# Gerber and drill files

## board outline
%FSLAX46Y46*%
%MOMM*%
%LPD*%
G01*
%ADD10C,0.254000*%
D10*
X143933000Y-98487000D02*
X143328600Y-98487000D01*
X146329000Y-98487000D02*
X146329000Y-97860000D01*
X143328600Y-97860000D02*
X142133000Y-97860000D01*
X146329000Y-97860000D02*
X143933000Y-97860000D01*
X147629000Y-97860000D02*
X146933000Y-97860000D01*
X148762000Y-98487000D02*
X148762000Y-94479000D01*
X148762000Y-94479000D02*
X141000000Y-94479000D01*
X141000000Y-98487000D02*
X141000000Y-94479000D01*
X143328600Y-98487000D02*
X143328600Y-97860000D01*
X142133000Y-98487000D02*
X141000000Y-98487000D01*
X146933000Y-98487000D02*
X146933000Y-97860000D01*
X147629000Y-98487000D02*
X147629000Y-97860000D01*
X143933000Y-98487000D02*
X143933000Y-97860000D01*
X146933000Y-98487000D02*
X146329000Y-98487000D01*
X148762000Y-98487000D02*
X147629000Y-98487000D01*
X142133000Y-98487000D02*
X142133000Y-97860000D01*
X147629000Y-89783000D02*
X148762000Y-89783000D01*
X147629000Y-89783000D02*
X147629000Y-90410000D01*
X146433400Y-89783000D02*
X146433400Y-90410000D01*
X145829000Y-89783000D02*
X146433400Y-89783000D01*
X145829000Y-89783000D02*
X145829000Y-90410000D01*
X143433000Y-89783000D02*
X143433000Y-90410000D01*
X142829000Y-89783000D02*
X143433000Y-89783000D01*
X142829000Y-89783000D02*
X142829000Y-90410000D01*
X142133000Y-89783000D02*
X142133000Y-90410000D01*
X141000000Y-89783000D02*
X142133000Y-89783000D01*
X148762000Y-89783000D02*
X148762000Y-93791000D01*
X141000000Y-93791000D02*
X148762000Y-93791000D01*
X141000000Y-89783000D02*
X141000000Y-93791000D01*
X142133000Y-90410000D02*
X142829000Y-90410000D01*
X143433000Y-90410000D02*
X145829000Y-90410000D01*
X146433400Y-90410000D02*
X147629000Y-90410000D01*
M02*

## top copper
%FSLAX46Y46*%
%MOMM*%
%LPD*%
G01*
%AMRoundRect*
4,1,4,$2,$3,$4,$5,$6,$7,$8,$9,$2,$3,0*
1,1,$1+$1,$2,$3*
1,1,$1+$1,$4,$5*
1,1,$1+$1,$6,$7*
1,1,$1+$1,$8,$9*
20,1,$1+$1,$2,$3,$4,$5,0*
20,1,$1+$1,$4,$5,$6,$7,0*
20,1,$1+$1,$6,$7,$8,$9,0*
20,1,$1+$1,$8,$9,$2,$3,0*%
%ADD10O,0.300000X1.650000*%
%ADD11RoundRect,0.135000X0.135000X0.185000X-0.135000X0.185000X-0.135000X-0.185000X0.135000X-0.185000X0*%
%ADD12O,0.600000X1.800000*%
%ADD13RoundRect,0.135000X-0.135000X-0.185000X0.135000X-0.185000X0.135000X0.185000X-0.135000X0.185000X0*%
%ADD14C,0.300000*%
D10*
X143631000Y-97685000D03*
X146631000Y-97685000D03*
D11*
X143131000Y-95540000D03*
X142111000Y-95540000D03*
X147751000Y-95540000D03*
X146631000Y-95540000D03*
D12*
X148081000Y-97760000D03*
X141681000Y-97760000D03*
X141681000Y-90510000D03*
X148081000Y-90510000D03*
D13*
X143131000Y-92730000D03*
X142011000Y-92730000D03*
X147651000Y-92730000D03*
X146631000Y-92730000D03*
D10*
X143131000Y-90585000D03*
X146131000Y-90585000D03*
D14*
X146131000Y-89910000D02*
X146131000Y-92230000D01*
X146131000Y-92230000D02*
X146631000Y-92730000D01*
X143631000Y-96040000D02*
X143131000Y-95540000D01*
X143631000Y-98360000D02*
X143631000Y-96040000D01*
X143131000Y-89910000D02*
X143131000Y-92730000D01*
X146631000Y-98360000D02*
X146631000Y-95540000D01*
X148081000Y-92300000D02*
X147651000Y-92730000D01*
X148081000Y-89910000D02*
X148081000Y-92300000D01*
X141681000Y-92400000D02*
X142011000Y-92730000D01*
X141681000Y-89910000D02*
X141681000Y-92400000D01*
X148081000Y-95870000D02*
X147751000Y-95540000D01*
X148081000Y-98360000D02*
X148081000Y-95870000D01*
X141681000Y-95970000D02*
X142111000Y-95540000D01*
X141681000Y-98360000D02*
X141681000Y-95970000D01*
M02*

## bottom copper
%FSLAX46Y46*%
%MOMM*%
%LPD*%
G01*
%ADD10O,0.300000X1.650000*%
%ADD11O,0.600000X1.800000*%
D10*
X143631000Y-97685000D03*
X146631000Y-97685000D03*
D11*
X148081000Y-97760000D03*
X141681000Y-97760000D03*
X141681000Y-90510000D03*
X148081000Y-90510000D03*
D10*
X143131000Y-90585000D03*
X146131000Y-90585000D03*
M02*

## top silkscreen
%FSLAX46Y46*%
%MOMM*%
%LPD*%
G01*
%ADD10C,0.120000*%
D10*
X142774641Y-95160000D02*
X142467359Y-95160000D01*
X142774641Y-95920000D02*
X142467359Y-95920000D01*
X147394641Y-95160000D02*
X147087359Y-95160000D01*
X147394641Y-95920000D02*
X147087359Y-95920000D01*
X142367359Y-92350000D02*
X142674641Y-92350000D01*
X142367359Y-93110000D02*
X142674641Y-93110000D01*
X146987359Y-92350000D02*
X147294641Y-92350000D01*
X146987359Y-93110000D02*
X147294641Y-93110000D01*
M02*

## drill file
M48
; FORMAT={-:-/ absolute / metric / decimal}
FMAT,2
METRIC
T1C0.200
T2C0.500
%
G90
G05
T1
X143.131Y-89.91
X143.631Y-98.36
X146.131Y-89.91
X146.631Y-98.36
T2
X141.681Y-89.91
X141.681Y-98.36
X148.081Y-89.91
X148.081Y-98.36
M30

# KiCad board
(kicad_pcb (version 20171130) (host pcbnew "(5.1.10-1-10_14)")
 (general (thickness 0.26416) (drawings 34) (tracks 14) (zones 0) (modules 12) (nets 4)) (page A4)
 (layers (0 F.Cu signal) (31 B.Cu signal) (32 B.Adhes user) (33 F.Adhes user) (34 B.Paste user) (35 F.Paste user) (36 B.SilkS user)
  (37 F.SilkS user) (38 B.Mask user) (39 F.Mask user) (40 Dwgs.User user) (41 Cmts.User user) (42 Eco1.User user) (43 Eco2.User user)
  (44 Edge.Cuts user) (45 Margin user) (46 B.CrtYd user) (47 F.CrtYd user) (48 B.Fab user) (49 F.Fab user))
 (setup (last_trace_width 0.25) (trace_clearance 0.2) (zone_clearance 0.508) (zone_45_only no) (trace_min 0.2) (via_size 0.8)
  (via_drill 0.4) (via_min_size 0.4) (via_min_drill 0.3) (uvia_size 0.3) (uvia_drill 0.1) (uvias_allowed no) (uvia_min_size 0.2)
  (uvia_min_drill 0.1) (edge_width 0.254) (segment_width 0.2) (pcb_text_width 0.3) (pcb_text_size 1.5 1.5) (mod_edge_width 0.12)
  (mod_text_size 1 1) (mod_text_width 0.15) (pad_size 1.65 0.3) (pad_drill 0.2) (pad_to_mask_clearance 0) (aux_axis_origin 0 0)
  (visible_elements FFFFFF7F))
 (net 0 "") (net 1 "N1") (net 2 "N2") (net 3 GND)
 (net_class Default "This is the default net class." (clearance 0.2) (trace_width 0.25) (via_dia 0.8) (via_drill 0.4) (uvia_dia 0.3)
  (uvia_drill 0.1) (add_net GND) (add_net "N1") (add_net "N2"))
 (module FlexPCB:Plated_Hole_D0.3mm (layer F.Cu) (at 142.941 95.36 90)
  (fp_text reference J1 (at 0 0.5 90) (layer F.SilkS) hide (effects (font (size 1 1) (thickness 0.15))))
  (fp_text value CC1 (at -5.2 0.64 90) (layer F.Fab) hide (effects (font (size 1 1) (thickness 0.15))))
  (pad A5 thru_hole oval (at -3 0.69 90) (size 1.65 0.3) (drill 0.2 (offset 0.675 0)) (layers *.Cu *.Mask) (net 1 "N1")))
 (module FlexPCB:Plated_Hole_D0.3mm (layer F.Cu) (at 149.161 95.36 90)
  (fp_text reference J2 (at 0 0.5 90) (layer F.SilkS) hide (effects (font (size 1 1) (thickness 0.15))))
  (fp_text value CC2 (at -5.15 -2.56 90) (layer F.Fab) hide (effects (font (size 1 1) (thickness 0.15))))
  (pad B5 thru_hole oval (at -3 -2.53 90) (size 1.65 0.3) (drill 0.2 (offset 0.675 0)) (layers *.Cu *.Mask) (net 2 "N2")))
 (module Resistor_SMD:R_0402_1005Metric (layer F.Cu) (at 142.621 95.54 180)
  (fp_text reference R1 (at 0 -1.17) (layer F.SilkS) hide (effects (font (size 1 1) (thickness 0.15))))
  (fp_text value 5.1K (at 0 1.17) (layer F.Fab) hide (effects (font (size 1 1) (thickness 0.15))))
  (fp_line (start -0.153641 0.38) (end 0.153641 0.38) (layer F.SilkS) (width 0.12))
  (fp_line (start -0.153641 -0.38) (end 0.153641 -0.38) (layer F.SilkS) (width 0.12))
  (pad 1 smd roundrect (at -0.51 0 180) (size 0.54 0.64) (layers F.Cu F.Paste F.Mask) (roundrect_rratio 0.25) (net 1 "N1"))
  (pad 2 smd roundrect (at 0.51 0 180) (size 0.54 0.64) (layers F.Cu F.Paste F.Mask) (roundrect_rratio 0.25) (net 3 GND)))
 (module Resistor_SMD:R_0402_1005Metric (layer F.Cu) (at 147.241 95.54 180)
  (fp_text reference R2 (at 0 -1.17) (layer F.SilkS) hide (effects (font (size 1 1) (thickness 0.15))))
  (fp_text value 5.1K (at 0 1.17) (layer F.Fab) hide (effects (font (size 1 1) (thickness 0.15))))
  (fp_line (start -0.153641 0.38) (end 0.153641 0.38) (layer F.SilkS) (width 0.12))
  (fp_line (start -0.153641 -0.38) (end 0.153641 -0.38) (layer F.SilkS) (width 0.12))
  (pad 1 smd roundrect (at -0.51 0 180) (size 0.54 0.64) (layers F.Cu F.Paste F.Mask) (roundrect_rratio 0.25) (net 3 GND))
  (pad 2 smd roundrect (at 0.61 0 180) (size 0.54 0.64) (layers F.Cu F.Paste F.Mask) (roundrect_rratio 0.25) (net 2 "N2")))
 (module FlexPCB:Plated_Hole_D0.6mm (layer F.Cu) (at 146.111 99.52 180)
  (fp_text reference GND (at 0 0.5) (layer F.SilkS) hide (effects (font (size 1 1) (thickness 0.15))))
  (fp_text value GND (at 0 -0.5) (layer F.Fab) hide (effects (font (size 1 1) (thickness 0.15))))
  (pad B1 thru_hole oval (at -1.97 1.16 90) (size 1.8 0.6) (drill 0.5 (offset 0.6 0)) (layers *.Cu *.Mask) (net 3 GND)))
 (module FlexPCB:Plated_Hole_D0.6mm (layer F.Cu) (at 138.771 99.66 180)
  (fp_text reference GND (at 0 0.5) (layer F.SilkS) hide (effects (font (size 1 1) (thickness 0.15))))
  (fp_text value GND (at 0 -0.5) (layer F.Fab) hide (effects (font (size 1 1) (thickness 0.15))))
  (pad A1 thru_hole oval (at -2.91 1.3 90) (size 1.8 0.6) (drill 0.5 (offset 0.6 0)) (layers *.Cu *.Mask) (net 3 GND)))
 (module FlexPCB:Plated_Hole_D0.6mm (layer F.Cu) (at 143.651 88.75)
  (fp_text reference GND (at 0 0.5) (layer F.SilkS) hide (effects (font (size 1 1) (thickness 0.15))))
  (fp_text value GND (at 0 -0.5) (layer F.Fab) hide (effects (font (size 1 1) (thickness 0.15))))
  (pad B1 thru_hole oval (at -1.97 1.16 270) (size 1.8 0.6) (drill 0.5 (offset 0.6 0)) (layers *.Cu *.Mask) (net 3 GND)))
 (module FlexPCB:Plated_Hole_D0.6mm (layer F.Cu) (at 150.991 88.61)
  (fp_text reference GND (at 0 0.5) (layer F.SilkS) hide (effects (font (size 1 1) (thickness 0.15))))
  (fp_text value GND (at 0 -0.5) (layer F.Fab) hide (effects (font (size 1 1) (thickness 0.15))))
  (pad A1 thru_hole oval (at -2.91 1.3 270) (size 1.8 0.6) (drill 0.5 (offset 0.6 0)) (layers *.Cu *.Mask) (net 3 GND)))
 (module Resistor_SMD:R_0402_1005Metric (layer F.Cu) (at 142.521 92.73)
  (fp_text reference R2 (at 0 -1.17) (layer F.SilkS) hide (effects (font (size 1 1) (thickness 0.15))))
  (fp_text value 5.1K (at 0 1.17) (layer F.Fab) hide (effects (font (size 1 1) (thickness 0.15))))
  (fp_line (start -0.153641 -0.38) (end 0.153641 -0.38) (layer F.SilkS) (width 0.12))
  (fp_line (start -0.153641 0.38) (end 0.153641 0.38) (layer F.SilkS) (width 0.12))
  (pad 2 smd roundrect (at 0.61 0) (size 0.54 0.64) (layers F.Cu F.Paste F.Mask) (roundrect_rratio 0.25) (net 2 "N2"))
  (pad 1 smd roundrect (at -0.51 0) (size 0.54 0.64) (layers F.Cu F.Paste F.Mask) (roundrect_rratio 0.25) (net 3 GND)))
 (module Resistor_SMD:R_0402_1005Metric (layer F.Cu) (at 147.141 92.73)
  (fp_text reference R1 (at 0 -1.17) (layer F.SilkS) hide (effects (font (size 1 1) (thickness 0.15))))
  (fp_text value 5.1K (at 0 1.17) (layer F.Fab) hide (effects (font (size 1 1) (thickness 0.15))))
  (fp_line (start -0.153641 -0.38) (end 0.153641 -0.38) (layer F.SilkS) (width 0.12))
  (fp_line (start -0.153641 0.38) (end 0.153641 0.38) (layer F.SilkS) (width 0.12))
  (pad 2 smd roundrect (at 0.51 0) (size 0.54 0.64) (layers F.Cu F.Paste F.Mask) (roundrect_rratio 0.25) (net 3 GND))
  (pad 1 smd roundrect (at -0.51 0) (size 0.54 0.64) (layers F.Cu F.Paste F.Mask) (roundrect_rratio 0.25) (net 1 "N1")))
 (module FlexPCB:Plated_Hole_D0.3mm (layer F.Cu) (at 140.601 92.91 270)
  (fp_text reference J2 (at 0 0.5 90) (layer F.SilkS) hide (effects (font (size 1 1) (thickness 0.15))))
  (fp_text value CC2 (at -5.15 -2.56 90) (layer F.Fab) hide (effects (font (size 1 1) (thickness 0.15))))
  (pad B5 thru_hole oval (at -3 -2.53 270) (size 1.65 0.3) (drill 0.2 (offset 0.675 0)) (layers *.Cu *.Mask) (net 2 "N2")))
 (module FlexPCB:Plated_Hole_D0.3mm (layer F.Cu) (at 146.821 92.91 270)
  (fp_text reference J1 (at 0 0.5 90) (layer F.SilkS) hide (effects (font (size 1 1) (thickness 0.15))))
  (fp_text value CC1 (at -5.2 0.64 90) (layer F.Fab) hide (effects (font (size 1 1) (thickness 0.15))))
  (pad A5 thru_hole oval (at -3 0.69 270) (size 1.65 0.3) (drill 0.2 (offset 0.675 0)) (layers *.Cu *.Mask) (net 1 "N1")))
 (gr_line (start 143.933 98.487) (end 143.3286 98.487) (layer Edge.Cuts) (width 0.254))
 (gr_line (start 146.329 98.487) (end 146.329 97.86) (layer Edge.Cuts) (width 0.254))
 (gr_line (start 143.3286 97.86) (end 142.133 97.86) (layer Edge.Cuts) (width 0.254))
 (gr_line (start 146.329 97.86) (end 143.933 97.86) (layer Edge.Cuts) (width 0.254))
 (gr_line (start 147.629 97.86) (end 146.933 97.86) (layer Edge.Cuts) (width 0.254))
 (gr_line (start 148.762 98.487) (end 148.762 94.479) (layer Edge.Cuts) (width 0.254))
 (gr_line (start 148.762 94.479) (end 141 94.479) (layer Edge.Cuts) (width 0.254))
 (gr_line (start 141 98.487) (end 141 94.479) (layer Edge.Cuts) (width 0.254))
 (gr_line (start 143.3286 98.487) (end 143.3286 97.86) (layer Edge.Cuts) (width 0.254))
 (gr_line (start 142.133 98.487) (end 141 98.487) (layer Edge.Cuts) (width 0.254))
 (gr_line (start 146.933 98.487) (end 146.933 97.86) (layer Edge.Cuts) (width 0.254))
 (gr_line (start 147.629 98.487) (end 147.629 97.86) (layer Edge.Cuts) (width 0.254))
 (gr_line (start 143.933 98.487) (end 143.933 97.86) (layer Edge.Cuts) (width 0.254))
 (gr_line (start 146.933 98.487) (end 146.329 98.487) (layer Edge.Cuts) (width 0.254))
 (gr_line (start 148.762 98.487) (end 147.629 98.487) (layer Edge.Cuts) (width 0.254))
 (gr_line (start 142.133 98.487) (end 142.133 97.86) (layer Edge.Cuts) (width 0.254))
 (gr_line (start 147.629 89.783) (end 148.762 89.783) (layer Edge.Cuts) (width 0.254))
 (gr_line (start 147.629 89.783) (end 147.629 90.41) (layer Edge.Cuts) (width 0.254))
 (gr_line (start 146.4334 89.783) (end 146.4334 90.41) (layer Edge.Cuts) (width 0.254))
 (gr_line (start 145.829 89.783) (end 146.4334 89.783) (layer Edge.Cuts) (width 0.254))
 (gr_line (start 145.829 89.783) (end 145.829 90.41) (layer Edge.Cuts) (width 0.254))
 (gr_line (start 143.433 89.783) (end 143.433 90.41) (layer Edge.Cuts) (width 0.254))
 (gr_line (start 142.829 89.783) (end 143.433 89.783) (layer Edge.Cuts) (width 0.254))
 (gr_line (start 142.829 89.783) (end 142.829 90.41) (layer Edge.Cuts) (width 0.254))
 (gr_line (start 142.133 89.783) (end 142.133 90.41) (layer Edge.Cuts) (width 0.254))
 (gr_line (start 141 89.783) (end 142.133 89.783) (layer Edge.Cuts) (width 0.254))
 (gr_line (start 148.762 89.783) (end 148.762 93.791) (layer Edge.Cuts) (width 0.254))
 (gr_line (start 141 93.791) (end 148.762 93.791) (layer Edge.Cuts) (width 0.254))
 (gr_line (start 141 89.783) (end 141 93.791) (layer Edge.Cuts) (width 0.254))
 (gr_line (start 142.133 90.41) (end 142.829 90.41) (layer Edge.Cuts) (width 0.254))
 (gr_line (start 143.433 90.41) (end 145.829 90.41) (layer Edge.Cuts) (width 0.254))
 (gr_line (start 146.4334 90.41) (end 147.629 90.41) (layer Edge.Cuts) (width 0.254))
 (segment (start 146.131 89.91) (end 146.131 92.23) (width 0.3) (layer F.Cu) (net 1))
 (segment (start 146.131 92.23) (end 146.631 92.73) (width 0.3) (layer F.Cu) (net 1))
 (segment (start 143.631 96.04) (end 143.131 95.54) (width 0.3) (layer F.Cu) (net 1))
 (segment (start 143.631 98.36) (end 143.631 96.04) (width 0.3) (layer F.Cu) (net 1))
 (segment (start 143.131 89.91) (end 143.131 92.73) (width 0.3) (layer F.Cu) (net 2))
 (segment (start 146.631 98.36) (end 146.631 95.54) (width 0.3) (layer F.Cu) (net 2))
 (segment (start 148.081 92.3) (end 147.651 92.73) (width 0.3) (layer F.Cu) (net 3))
 (segment (start 148.081 89.91) (end 148.081 92.3) (width 0.3) (layer F.Cu) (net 3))
 (segment (start 141.681 92.4) (end 142.011 92.73) (width 0.3) (layer F.Cu) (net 3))
 (segment (start 141.681 89.91) (end 141.681 92.4) (width 0.3) (layer F.Cu) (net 3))
 (segment (start 148.081 95.87) (end 147.751 95.54) (width 0.3) (layer F.Cu) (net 3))
 (segment (start 148.081 98.36) (end 148.081 95.87) (width 0.3) (layer F.Cu) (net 3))
 (segment (start 141.681 95.97) (end 142.111 95.54) (width 0.3) (layer F.Cu) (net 3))
 (segment (start 141.681 98.36) (end 141.681 95.97) (width 0.3) (layer F.Cu) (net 3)))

